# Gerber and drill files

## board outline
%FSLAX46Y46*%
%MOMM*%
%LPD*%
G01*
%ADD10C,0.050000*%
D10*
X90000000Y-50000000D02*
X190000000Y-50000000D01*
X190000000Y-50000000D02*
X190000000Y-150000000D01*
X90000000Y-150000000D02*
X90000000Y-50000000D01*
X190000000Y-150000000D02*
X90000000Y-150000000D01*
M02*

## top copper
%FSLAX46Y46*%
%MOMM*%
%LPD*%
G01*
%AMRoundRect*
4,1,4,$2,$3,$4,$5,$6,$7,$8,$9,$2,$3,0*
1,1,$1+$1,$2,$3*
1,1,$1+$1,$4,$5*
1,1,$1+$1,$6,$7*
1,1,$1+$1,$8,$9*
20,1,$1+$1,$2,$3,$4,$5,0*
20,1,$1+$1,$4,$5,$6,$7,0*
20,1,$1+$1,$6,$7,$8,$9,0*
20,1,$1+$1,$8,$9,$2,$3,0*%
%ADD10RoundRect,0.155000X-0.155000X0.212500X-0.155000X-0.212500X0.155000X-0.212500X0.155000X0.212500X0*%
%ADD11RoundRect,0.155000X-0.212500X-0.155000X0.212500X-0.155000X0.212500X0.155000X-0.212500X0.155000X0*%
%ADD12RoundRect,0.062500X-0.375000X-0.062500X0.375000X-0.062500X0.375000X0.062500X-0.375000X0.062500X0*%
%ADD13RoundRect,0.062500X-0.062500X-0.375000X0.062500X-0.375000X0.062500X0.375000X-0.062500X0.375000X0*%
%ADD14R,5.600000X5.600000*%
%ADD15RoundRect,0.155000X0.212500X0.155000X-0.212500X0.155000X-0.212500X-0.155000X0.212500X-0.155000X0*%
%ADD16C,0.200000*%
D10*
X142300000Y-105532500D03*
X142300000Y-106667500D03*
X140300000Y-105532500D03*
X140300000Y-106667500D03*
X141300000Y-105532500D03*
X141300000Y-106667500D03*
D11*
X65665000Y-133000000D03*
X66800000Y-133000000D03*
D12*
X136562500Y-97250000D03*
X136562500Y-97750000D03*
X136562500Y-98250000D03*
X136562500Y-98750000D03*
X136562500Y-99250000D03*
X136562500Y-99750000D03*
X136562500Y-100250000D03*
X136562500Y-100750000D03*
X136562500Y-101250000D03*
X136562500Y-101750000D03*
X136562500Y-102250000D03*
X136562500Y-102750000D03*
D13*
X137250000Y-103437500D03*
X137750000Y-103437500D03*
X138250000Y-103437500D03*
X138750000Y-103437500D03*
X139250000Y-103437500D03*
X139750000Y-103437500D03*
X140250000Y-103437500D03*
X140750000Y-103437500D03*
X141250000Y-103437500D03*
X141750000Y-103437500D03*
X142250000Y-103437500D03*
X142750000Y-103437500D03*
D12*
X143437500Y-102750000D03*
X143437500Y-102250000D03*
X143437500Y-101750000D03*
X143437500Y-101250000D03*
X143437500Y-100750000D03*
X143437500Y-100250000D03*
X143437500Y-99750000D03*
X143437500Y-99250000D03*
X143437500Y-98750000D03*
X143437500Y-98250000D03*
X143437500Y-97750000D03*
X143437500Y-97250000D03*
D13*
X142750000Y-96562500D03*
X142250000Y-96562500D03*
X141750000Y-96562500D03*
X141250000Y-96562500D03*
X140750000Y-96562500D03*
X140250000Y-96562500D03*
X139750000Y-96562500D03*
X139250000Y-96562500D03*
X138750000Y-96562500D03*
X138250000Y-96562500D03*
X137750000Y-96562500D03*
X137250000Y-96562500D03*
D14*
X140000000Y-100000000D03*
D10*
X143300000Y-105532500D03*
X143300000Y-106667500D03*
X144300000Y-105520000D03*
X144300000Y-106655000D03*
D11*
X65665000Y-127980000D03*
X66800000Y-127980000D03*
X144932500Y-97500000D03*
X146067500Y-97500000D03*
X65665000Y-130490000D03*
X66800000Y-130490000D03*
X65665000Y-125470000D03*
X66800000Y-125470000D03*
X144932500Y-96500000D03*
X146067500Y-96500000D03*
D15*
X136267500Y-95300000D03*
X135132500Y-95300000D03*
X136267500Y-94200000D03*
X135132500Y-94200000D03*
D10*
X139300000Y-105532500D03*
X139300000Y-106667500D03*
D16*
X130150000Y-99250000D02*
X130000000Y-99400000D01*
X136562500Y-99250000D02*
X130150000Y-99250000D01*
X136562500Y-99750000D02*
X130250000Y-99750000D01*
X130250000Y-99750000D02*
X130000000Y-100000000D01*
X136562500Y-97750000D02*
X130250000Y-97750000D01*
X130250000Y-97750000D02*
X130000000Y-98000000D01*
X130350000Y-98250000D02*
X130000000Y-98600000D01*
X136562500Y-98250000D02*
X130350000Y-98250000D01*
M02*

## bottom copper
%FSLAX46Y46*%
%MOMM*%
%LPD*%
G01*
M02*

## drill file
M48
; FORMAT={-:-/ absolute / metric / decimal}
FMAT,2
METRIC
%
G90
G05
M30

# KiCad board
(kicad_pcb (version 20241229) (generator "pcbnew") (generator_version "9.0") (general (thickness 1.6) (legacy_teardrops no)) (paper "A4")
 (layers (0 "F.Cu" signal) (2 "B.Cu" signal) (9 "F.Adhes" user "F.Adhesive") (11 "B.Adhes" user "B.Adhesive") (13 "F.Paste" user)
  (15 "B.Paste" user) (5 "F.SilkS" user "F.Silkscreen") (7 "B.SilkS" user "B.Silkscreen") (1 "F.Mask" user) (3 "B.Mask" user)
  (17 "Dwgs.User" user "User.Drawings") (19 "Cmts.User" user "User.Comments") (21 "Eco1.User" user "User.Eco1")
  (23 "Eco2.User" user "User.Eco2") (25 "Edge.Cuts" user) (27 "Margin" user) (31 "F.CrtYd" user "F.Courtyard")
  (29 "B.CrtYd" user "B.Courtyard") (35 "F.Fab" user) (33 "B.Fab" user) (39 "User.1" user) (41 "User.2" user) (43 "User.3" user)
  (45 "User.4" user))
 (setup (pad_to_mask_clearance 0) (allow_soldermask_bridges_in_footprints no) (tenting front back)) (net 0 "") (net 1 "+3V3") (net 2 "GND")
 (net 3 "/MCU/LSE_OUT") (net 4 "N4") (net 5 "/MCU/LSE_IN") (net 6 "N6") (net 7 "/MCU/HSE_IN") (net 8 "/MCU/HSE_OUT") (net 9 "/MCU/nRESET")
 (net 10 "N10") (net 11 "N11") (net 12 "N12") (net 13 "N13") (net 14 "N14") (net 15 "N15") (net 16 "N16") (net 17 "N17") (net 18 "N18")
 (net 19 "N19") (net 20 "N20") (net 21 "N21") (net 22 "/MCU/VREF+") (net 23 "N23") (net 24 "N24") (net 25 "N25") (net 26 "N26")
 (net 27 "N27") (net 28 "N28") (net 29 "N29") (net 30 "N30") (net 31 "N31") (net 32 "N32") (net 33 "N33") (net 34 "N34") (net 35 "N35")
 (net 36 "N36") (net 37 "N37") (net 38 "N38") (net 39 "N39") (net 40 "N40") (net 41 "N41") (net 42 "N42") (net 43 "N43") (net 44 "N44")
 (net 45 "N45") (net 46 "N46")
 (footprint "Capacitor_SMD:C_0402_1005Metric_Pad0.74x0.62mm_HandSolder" (layer "F.Cu") (at 142.3 106.1 -90)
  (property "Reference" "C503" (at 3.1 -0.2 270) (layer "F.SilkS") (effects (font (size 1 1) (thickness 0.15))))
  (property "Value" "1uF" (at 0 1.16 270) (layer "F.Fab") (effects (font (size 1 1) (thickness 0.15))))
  (pad "1" smd roundrect (at -0.5675 0 270) (size 0.735 0.62) (layers "F.Cu" "F.Mask" "F.Paste") (roundrect_rratio 0.25) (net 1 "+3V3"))
  (pad "2" smd roundrect (at 0.5675 0 270) (size 0.735 0.62) (layers "F.Cu" "F.Mask" "F.Paste") (roundrect_rratio 0.25) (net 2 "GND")))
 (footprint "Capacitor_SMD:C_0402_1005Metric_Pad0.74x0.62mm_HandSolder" (layer "F.Cu") (at 140.3 106.1 -90)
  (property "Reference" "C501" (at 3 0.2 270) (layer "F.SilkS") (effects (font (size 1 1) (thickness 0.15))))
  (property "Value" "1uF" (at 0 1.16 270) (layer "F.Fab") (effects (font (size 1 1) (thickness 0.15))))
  (pad "1" smd roundrect (at -0.5675 0 270) (size 0.735 0.62) (layers "F.Cu" "F.Mask" "F.Paste") (roundrect_rratio 0.25) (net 1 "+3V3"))
  (pad "2" smd roundrect (at 0.5675 0 270) (size 0.735 0.62) (layers "F.Cu" "F.Mask" "F.Paste") (roundrect_rratio 0.25) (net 2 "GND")))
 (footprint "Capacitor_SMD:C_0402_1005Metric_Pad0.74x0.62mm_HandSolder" (layer "F.Cu") (at 141.3 106.1 -90)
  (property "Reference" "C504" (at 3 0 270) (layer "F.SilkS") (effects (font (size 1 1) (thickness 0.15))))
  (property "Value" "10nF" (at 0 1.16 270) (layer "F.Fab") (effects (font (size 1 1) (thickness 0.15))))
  (pad "1" smd roundrect (at -0.5675 0 270) (size 0.735 0.62) (layers "F.Cu" "F.Mask" "F.Paste") (roundrect_rratio 0.25) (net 1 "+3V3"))
  (pad "2" smd roundrect (at 0.5675 0 270) (size 0.735 0.62) (layers "F.Cu" "F.Mask" "F.Paste") (roundrect_rratio 0.25) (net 2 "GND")))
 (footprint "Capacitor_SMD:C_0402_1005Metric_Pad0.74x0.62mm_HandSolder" (layer "F.Cu") (at 66.2325 133)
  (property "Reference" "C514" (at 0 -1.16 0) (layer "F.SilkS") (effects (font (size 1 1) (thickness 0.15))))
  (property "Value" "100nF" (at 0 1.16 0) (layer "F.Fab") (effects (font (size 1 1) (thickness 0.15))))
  (pad "1" smd roundrect (at -0.5675 0) (size 0.735 0.62) (layers "F.Cu" "F.Mask" "F.Paste") (roundrect_rratio 0.25) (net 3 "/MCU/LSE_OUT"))
  (pad "2" smd roundrect (at 0.5675 0) (size 0.735 0.62) (layers "F.Cu" "F.Mask" "F.Paste") (roundrect_rratio 0.25) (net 2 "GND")))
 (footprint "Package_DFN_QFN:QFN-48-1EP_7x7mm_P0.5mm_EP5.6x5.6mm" (layer "F.Cu") (at 140 100)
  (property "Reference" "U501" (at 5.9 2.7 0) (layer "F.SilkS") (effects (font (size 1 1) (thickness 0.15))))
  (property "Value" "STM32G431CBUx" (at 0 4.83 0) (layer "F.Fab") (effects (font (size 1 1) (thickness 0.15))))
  (pad "" smd roundrect (at -2.1 -2.1) (size 1.13 1.13) (layers "F.Paste") (roundrect_rratio 0.221239))
  (pad "" smd roundrect (at -2.1 -0.7) (size 1.13 1.13) (layers "F.Paste") (roundrect_rratio 0.221239))
  (pad "" smd roundrect (at -2.1 0.7) (size 1.13 1.13) (layers "F.Paste") (roundrect_rratio 0.221239))
  (pad "" smd roundrect (at -2.1 2.1) (size 1.13 1.13) (layers "F.Paste") (roundrect_rratio 0.221239))
  (pad "" smd roundrect (at -0.7 -2.1) (size 1.13 1.13) (layers "F.Paste") (roundrect_rratio 0.221239))
  (pad "" smd roundrect (at -0.7 -0.7) (size 1.13 1.13) (layers "F.Paste") (roundrect_rratio 0.221239))
  (pad "" smd roundrect (at -0.7 0.7) (size 1.13 1.13) (layers "F.Paste") (roundrect_rratio 0.221239))
  (pad "" smd roundrect (at -0.7 2.1) (size 1.13 1.13) (layers "F.Paste") (roundrect_rratio 0.221239))
  (pad "" smd roundrect (at 0.7 -2.1) (size 1.13 1.13) (layers "F.Paste") (roundrect_rratio 0.221239))
  (pad "" smd roundrect (at 0.7 -0.7) (size 1.13 1.13) (layers "F.Paste") (roundrect_rratio 0.221239))
  (pad "" smd roundrect (at 0.7 0.7) (size 1.13 1.13) (layers "F.Paste") (roundrect_rratio 0.221239))
  (pad "" smd roundrect (at 0.7 2.1) (size 1.13 1.13) (layers "F.Paste") (roundrect_rratio 0.221239))
  (pad "" smd roundrect (at 2.1 -2.1) (size 1.13 1.13) (layers "F.Paste") (roundrect_rratio 0.221239))
  (pad "" smd roundrect (at 2.1 -0.7) (size 1.13 1.13) (layers "F.Paste") (roundrect_rratio 0.221239))
  (pad "" smd roundrect (at 2.1 0.7) (size 1.13 1.13) (layers "F.Paste") (roundrect_rratio 0.221239))
  (pad "" smd roundrect (at 2.1 2.1) (size 1.13 1.13) (layers "F.Paste") (roundrect_rratio 0.221239))
  (pad "1" smd roundrect (at -3.4375 -2.75) (size 0.875 0.25) (layers "F.Cu" "F.Mask" "F.Paste") (roundrect_rratio 0.25) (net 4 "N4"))
  (pad "2" smd roundrect (at -3.4375 -2.25) (size 0.875 0.25) (layers "F.Cu" "F.Mask" "F.Paste") (roundrect_rratio 0.25)
   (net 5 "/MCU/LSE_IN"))
  (pad "3" smd roundrect (at -3.4375 -1.75) (size 0.875 0.25) (layers "F.Cu" "F.Mask" "F.Paste") (roundrect_rratio 0.25)
   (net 3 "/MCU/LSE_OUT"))
  (pad "4" smd roundrect (at -3.4375 -1.25) (size 0.875 0.25) (layers "F.Cu" "F.Mask" "F.Paste") (roundrect_rratio 0.25) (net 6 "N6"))
  (pad "5" smd roundrect (at -3.4375 -0.75) (size 0.875 0.25) (layers "F.Cu" "F.Mask" "F.Paste") (roundrect_rratio 0.25)
   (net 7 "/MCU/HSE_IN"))
  (pad "6" smd roundrect (at -3.4375 -0.25) (size 0.875 0.25) (layers "F.Cu" "F.Mask" "F.Paste") (roundrect_rratio 0.25)
   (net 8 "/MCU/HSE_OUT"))
  (pad "7" smd roundrect (at -3.4375 0.25) (size 0.875 0.25) (layers "F.Cu" "F.Mask" "F.Paste") (roundrect_rratio 0.25)
   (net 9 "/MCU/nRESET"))
  (pad "8" smd roundrect (at -3.4375 0.75) (size 0.875 0.25) (layers "F.Cu" "F.Mask" "F.Paste") (roundrect_rratio 0.25) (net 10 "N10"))
  (pad "9" smd roundrect (at -3.4375 1.25) (size 0.875 0.25) (layers "F.Cu" "F.Mask" "F.Paste") (roundrect_rratio 0.25) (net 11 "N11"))
  (pad "10" smd roundrect (at -3.4375 1.75) (size 0.875 0.25) (layers "F.Cu" "F.Mask" "F.Paste") (roundrect_rratio 0.25) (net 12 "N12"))
  (pad "11" smd roundrect (at -3.4375 2.25) (size 0.875 0.25) (layers "F.Cu" "F.Mask" "F.Paste") (roundrect_rratio 0.25) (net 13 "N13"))
  (pad "12" smd roundrect (at -3.4375 2.75) (size 0.875 0.25) (layers "F.Cu" "F.Mask" "F.Paste") (roundrect_rratio 0.25) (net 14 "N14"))
  (pad "13" smd roundrect (at -2.75 3.4375) (size 0.25 0.875) (layers "F.Cu" "F.Mask" "F.Paste") (roundrect_rratio 0.25) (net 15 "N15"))
  (pad "14" smd roundrect (at -2.25 3.4375) (size 0.25 0.875) (layers "F.Cu" "F.Mask" "F.Paste") (roundrect_rratio 0.25) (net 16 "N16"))
  (pad "15" smd roundrect (at -1.75 3.4375) (size 0.25 0.875) (layers "F.Cu" "F.Mask" "F.Paste") (roundrect_rratio 0.25) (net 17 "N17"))
  (pad "16" smd roundrect (at -1.25 3.4375) (size 0.25 0.875) (layers "F.Cu" "F.Mask" "F.Paste") (roundrect_rratio 0.25) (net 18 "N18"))
  (pad "17" smd roundrect (at -0.75 3.4375) (size 0.25 0.875) (layers "F.Cu" "F.Mask" "F.Paste") (roundrect_rratio 0.25) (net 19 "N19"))
  (pad "18" smd roundrect (at -0.25 3.4375) (size 0.25 0.875) (layers "F.Cu" "F.Mask" "F.Paste") (roundrect_rratio 0.25) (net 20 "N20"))
  (pad "19" smd roundrect (at 0.25 3.4375) (size 0.25 0.875) (layers "F.Cu" "F.Mask" "F.Paste") (roundrect_rratio 0.25) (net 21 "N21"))
  (pad "20" smd roundrect (at 0.75 3.4375) (size 0.25 0.875) (layers "F.Cu" "F.Mask" "F.Paste") (roundrect_rratio 0.25)
   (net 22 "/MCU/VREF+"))
  (pad "21" smd roundrect (at 1.25 3.4375) (size 0.25 0.875) (layers "F.Cu" "F.Mask" "F.Paste") (roundrect_rratio 0.25) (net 1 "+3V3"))
  (pad "22" smd roundrect (at 1.75 3.4375) (size 0.25 0.875) (layers "F.Cu" "F.Mask" "F.Paste") (roundrect_rratio 0.25) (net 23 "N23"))
  (pad "23" smd roundrect (at 2.25 3.4375) (size 0.25 0.875) (layers "F.Cu" "F.Mask" "F.Paste") (roundrect_rratio 0.25) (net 1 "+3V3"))
  (pad "24" smd roundrect (at 2.75 3.4375) (size 0.25 0.875) (layers "F.Cu" "F.Mask" "F.Paste") (roundrect_rratio 0.25) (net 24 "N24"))
  (pad "25" smd roundrect (at 3.4375 2.75) (size 0.875 0.25) (layers "F.Cu" "F.Mask" "F.Paste") (roundrect_rratio 0.25) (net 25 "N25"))
  (pad "26" smd roundrect (at 3.4375 2.25) (size 0.875 0.25) (layers "F.Cu" "F.Mask" "F.Paste") (roundrect_rratio 0.25) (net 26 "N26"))
  (pad "27" smd roundrect (at 3.4375 1.75) (size 0.875 0.25) (layers "F.Cu" "F.Mask" "F.Paste") (roundrect_rratio 0.25) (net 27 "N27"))
  (pad "28" smd roundrect (at 3.4375 1.25) (size 0.875 0.25) (layers "F.Cu" "F.Mask" "F.Paste") (roundrect_rratio 0.25) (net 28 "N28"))
  (pad "29" smd roundrect (at 3.4375 0.75) (size 0.875 0.25) (layers "F.Cu" "F.Mask" "F.Paste") (roundrect_rratio 0.25) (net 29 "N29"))
  (pad "30" smd roundrect (at 3.4375 0.25) (size 0.875 0.25) (layers "F.Cu" "F.Mask" "F.Paste") (roundrect_rratio 0.25) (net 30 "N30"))
  (pad "31" smd roundrect (at 3.4375 -0.25) (size 0.875 0.25) (layers "F.Cu" "F.Mask" "F.Paste") (roundrect_rratio 0.25) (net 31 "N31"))
  (pad "32" smd roundrect (at 3.4375 -0.75) (size 0.875 0.25) (layers "F.Cu" "F.Mask" "F.Paste") (roundrect_rratio 0.25) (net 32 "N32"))
  (pad "33" smd roundrect (at 3.4375 -1.25) (size 0.875 0.25) (layers "F.Cu" "F.Mask" "F.Paste") (roundrect_rratio 0.25) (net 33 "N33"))
  (pad "34" smd roundrect (at 3.4375 -1.75) (size 0.875 0.25) (layers "F.Cu" "F.Mask" "F.Paste") (roundrect_rratio 0.25) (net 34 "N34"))
  (pad "35" smd roundrect (at 3.4375 -2.25) (size 0.875 0.25) (layers "F.Cu" "F.Mask" "F.Paste") (roundrect_rratio 0.25) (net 1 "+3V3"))
  (pad "36" smd roundrect (at 3.4375 -2.75) (size 0.875 0.25) (layers "F.Cu" "F.Mask" "F.Paste") (roundrect_rratio 0.25) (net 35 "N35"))
  (pad "37" smd roundrect (at 2.75 -3.4375) (size 0.25 0.875) (layers "F.Cu" "F.Mask" "F.Paste") (roundrect_rratio 0.25) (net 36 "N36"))
  (pad "38" smd roundrect (at 2.25 -3.4375) (size 0.25 0.875) (layers "F.Cu" "F.Mask" "F.Paste") (roundrect_rratio 0.25) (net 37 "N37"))
  (pad "39" smd roundrect (at 1.75 -3.4375) (size 0.25 0.875) (layers "F.Cu" "F.Mask" "F.Paste") (roundrect_rratio 0.25) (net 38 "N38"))
  (pad "40" smd roundrect (at 1.25 -3.4375) (size 0.25 0.875) (layers "F.Cu" "F.Mask" "F.Paste") (roundrect_rratio 0.25) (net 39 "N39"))
  (pad "41" smd roundrect (at 0.75 -3.4375) (size 0.25 0.875) (layers "F.Cu" "F.Mask" "F.Paste") (roundrect_rratio 0.25) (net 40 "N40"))
  (pad "42" smd roundrect (at 0.25 -3.4375) (size 0.25 0.875) (layers "F.Cu" "F.Mask" "F.Paste") (roundrect_rratio 0.25) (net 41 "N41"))
  (pad "43" smd roundrect (at -0.25 -3.4375) (size 0.25 0.875) (layers "F.Cu" "F.Mask" "F.Paste") (roundrect_rratio 0.25) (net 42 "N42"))
  (pad "44" smd roundrect (at -0.75 -3.4375) (size 0.25 0.875) (layers "F.Cu" "F.Mask" "F.Paste") (roundrect_rratio 0.25) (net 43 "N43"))
  (pad "45" smd roundrect (at -1.25 -3.4375) (size 0.25 0.875) (layers "F.Cu" "F.Mask" "F.Paste") (roundrect_rratio 0.25) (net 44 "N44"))
  (pad "46" smd roundrect (at -1.75 -3.4375) (size 0.25 0.875) (layers "F.Cu" "F.Mask" "F.Paste") (roundrect_rratio 0.25) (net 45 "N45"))
  (pad "47" smd roundrect (at -2.25 -3.4375) (size 0.25 0.875) (layers "F.Cu" "F.Mask" "F.Paste") (roundrect_rratio 0.25) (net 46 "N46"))
  (pad "48" smd roundrect (at -2.75 -3.4375) (size 0.25 0.875) (layers "F.Cu" "F.Mask" "F.Paste") (roundrect_rratio 0.25) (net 1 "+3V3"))
  (pad "49" smd rect (at 0 0) (size 5.6 5.6) (layers "F.Cu" "F.Mask") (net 2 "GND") (zone_connect 2)))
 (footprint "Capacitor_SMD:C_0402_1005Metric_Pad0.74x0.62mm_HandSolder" (layer "F.Cu") (at 143.3 106.1 -90)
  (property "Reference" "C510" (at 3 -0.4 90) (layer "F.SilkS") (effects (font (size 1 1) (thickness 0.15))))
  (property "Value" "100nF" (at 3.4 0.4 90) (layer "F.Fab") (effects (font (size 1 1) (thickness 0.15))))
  (pad "1" smd roundrect (at -0.5675 0 270) (size 0.735 0.62) (layers "F.Cu" "F.Mask" "F.Paste") (roundrect_rratio 0.25) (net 1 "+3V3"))
  (pad "2" smd roundrect (at 0.5675 0 270) (size 0.735 0.62) (layers "F.Cu" "F.Mask" "F.Paste") (roundrect_rratio 0.25) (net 2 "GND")))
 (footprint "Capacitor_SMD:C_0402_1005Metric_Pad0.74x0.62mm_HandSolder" (layer "F.Cu") (at 144.3 106.0875 -90)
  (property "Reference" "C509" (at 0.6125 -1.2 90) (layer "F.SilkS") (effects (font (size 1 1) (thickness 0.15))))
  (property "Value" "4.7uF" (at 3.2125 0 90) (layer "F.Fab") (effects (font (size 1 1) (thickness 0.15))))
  (pad "1" smd roundrect (at -0.5675 0 270) (size 0.735 0.62) (layers "F.Cu" "F.Mask" "F.Paste") (roundrect_rratio 0.25) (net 1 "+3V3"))
  (pad "2" smd roundrect (at 0.5675 0 270) (size 0.735 0.62) (layers "F.Cu" "F.Mask" "F.Paste") (roundrect_rratio 0.25) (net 2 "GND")))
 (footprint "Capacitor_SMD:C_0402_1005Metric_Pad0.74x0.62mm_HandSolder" (layer "F.Cu") (at 66.2325 127.98)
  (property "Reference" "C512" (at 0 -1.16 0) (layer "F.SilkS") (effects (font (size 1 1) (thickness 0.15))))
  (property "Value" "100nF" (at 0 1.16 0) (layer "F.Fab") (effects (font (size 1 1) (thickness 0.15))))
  (pad "1" smd roundrect (at -0.5675 0) (size 0.735 0.62) (layers "F.Cu" "F.Mask" "F.Paste") (roundrect_rratio 0.25) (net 8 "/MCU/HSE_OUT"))
  (pad "2" smd roundrect (at 0.5675 0) (size 0.735 0.62) (layers "F.Cu" "F.Mask" "F.Paste") (roundrect_rratio 0.25) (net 2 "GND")))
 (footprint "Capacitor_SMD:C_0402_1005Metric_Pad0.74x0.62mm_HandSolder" (layer "F.Cu") (at 145.5 97.5)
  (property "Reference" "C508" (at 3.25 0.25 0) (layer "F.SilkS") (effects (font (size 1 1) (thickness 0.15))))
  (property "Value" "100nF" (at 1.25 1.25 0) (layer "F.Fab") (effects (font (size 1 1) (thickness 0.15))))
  (pad "1" smd roundrect (at -0.5675 0) (size 0.735 0.62) (layers "F.Cu" "F.Mask" "F.Paste") (roundrect_rratio 0.25) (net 1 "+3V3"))
  (pad "2" smd roundrect (at 0.5675 0) (size 0.735 0.62) (layers "F.Cu" "F.Mask" "F.Paste") (roundrect_rratio 0.25) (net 2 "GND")))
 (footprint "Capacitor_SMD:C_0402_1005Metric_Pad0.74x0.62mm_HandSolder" (layer "F.Cu") (at 66.2325 130.49)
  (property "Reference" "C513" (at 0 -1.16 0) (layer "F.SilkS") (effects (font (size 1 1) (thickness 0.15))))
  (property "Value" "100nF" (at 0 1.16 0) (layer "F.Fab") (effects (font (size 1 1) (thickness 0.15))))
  (pad "1" smd roundrect (at -0.5675 0) (size 0.735 0.62) (layers "F.Cu" "F.Mask" "F.Paste") (roundrect_rratio 0.25) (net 5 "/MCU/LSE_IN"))
  (pad "2" smd roundrect (at 0.5675 0) (size 0.735 0.62) (layers "F.Cu" "F.Mask" "F.Paste") (roundrect_rratio 0.25) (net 2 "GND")))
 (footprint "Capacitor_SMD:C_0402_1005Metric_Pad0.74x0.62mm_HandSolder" (layer "F.Cu") (at 66.2325 125.47)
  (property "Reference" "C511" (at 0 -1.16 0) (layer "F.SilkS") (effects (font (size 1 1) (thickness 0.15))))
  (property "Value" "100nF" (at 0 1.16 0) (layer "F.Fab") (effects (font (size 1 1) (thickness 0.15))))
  (pad "1" smd roundrect (at -0.5675 0) (size 0.735 0.62) (layers "F.Cu" "F.Mask" "F.Paste") (roundrect_rratio 0.25) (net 7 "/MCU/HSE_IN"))
  (pad "2" smd roundrect (at 0.5675 0) (size 0.735 0.62) (layers "F.Cu" "F.Mask" "F.Paste") (roundrect_rratio 0.25) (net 2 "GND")))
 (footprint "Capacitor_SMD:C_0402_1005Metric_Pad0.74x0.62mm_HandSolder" (layer "F.Cu") (at 145.5 96.5)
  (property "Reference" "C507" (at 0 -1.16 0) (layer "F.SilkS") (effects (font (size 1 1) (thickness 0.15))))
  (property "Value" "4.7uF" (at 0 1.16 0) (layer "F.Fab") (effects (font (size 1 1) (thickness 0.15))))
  (pad "1" smd roundrect (at -0.5675 0) (size 0.735 0.62) (layers "F.Cu" "F.Mask" "F.Paste") (roundrect_rratio 0.25) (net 1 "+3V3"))
  (pad "2" smd roundrect (at 0.5675 0) (size 0.735 0.62) (layers "F.Cu" "F.Mask" "F.Paste") (roundrect_rratio 0.25) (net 2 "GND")))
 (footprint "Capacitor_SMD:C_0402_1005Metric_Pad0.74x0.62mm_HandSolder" (layer "F.Cu") (at 135.7 95.3 180)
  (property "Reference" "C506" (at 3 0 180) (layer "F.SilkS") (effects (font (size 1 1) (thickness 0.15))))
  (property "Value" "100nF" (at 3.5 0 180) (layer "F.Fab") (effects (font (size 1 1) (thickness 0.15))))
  (pad "1" smd roundrect (at -0.5675 0 180) (size 0.735 0.62) (layers "F.Cu" "F.Mask" "F.Paste") (roundrect_rratio 0.25) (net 1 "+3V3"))
  (pad "2" smd roundrect (at 0.5675 0 180) (size 0.735 0.62) (layers "F.Cu" "F.Mask" "F.Paste") (roundrect_rratio 0.25) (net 2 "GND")))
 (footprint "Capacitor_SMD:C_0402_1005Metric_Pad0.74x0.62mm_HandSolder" (layer "F.Cu") (at 135.7 94.2 180)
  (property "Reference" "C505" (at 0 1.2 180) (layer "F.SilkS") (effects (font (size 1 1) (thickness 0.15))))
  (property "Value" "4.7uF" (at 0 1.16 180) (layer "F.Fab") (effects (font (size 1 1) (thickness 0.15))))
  (pad "1" smd roundrect (at -0.5675 0 180) (size 0.735 0.62) (layers "F.Cu" "F.Mask" "F.Paste") (roundrect_rratio 0.25) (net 1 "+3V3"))
  (pad "2" smd roundrect (at 0.5675 0 180) (size 0.735 0.62) (layers "F.Cu" "F.Mask" "F.Paste") (roundrect_rratio 0.25) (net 2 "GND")))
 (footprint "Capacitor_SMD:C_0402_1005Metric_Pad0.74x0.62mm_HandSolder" (layer "F.Cu") (at 139.3 106.1 -90)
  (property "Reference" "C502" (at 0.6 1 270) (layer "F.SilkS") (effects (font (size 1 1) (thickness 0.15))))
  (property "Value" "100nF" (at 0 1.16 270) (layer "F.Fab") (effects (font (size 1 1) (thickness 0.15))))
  (pad "1" smd roundrect (at -0.5675 0 270) (size 0.735 0.62) (layers "F.Cu" "F.Mask" "F.Paste") (roundrect_rratio 0.25) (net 1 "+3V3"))
  (pad "2" smd roundrect (at 0.5675 0 270) (size 0.735 0.62) (layers "F.Cu" "F.Mask" "F.Paste") (roundrect_rratio 0.25) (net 2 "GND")))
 (gr_line (start 90 50) (end 190 50) (stroke (width 0.05) (type default)) (layer "Edge.Cuts"))
 (gr_line (start 190 50) (end 190 150) (stroke (width 0.05) (type default)) (layer "Edge.Cuts"))
 (gr_line (start 90 150) (end 90 50) (stroke (width 0.05) (type default)) (layer "Edge.Cuts"))
 (gr_line (start 190 150) (end 90 150) (stroke (width 0.05) (type default)) (layer "Edge.Cuts"))
 (segment (start 130.15 99.25) (end 130 99.4) (width 0.2) (layer "F.Cu") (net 7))
 (segment (start 136.5625 99.25) (end 130.15 99.25) (width 0.2) (layer "F.Cu") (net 7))
 (segment (start 136.5625 99.75) (end 130.25 99.75) (width 0.2) (layer "F.Cu") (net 8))
 (segment (start 130.25 99.75) (end 130 100) (width 0.2) (layer "F.Cu") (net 8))
 (segment (start 136.5625 97.75) (end 130.25 97.75) (width 0.2) (layer "F.Cu") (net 5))
 (segment (start 130.25 97.75) (end 130 98) (width 0.2) (layer "F.Cu") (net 5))
 (segment (start 130.35 98.25) (end 130 98.6) (width 0.2) (layer "F.Cu") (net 3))
 (segment (start 136.5625 98.25) (end 130.35 98.25) (width 0.2) (layer "F.Cu") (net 3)))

